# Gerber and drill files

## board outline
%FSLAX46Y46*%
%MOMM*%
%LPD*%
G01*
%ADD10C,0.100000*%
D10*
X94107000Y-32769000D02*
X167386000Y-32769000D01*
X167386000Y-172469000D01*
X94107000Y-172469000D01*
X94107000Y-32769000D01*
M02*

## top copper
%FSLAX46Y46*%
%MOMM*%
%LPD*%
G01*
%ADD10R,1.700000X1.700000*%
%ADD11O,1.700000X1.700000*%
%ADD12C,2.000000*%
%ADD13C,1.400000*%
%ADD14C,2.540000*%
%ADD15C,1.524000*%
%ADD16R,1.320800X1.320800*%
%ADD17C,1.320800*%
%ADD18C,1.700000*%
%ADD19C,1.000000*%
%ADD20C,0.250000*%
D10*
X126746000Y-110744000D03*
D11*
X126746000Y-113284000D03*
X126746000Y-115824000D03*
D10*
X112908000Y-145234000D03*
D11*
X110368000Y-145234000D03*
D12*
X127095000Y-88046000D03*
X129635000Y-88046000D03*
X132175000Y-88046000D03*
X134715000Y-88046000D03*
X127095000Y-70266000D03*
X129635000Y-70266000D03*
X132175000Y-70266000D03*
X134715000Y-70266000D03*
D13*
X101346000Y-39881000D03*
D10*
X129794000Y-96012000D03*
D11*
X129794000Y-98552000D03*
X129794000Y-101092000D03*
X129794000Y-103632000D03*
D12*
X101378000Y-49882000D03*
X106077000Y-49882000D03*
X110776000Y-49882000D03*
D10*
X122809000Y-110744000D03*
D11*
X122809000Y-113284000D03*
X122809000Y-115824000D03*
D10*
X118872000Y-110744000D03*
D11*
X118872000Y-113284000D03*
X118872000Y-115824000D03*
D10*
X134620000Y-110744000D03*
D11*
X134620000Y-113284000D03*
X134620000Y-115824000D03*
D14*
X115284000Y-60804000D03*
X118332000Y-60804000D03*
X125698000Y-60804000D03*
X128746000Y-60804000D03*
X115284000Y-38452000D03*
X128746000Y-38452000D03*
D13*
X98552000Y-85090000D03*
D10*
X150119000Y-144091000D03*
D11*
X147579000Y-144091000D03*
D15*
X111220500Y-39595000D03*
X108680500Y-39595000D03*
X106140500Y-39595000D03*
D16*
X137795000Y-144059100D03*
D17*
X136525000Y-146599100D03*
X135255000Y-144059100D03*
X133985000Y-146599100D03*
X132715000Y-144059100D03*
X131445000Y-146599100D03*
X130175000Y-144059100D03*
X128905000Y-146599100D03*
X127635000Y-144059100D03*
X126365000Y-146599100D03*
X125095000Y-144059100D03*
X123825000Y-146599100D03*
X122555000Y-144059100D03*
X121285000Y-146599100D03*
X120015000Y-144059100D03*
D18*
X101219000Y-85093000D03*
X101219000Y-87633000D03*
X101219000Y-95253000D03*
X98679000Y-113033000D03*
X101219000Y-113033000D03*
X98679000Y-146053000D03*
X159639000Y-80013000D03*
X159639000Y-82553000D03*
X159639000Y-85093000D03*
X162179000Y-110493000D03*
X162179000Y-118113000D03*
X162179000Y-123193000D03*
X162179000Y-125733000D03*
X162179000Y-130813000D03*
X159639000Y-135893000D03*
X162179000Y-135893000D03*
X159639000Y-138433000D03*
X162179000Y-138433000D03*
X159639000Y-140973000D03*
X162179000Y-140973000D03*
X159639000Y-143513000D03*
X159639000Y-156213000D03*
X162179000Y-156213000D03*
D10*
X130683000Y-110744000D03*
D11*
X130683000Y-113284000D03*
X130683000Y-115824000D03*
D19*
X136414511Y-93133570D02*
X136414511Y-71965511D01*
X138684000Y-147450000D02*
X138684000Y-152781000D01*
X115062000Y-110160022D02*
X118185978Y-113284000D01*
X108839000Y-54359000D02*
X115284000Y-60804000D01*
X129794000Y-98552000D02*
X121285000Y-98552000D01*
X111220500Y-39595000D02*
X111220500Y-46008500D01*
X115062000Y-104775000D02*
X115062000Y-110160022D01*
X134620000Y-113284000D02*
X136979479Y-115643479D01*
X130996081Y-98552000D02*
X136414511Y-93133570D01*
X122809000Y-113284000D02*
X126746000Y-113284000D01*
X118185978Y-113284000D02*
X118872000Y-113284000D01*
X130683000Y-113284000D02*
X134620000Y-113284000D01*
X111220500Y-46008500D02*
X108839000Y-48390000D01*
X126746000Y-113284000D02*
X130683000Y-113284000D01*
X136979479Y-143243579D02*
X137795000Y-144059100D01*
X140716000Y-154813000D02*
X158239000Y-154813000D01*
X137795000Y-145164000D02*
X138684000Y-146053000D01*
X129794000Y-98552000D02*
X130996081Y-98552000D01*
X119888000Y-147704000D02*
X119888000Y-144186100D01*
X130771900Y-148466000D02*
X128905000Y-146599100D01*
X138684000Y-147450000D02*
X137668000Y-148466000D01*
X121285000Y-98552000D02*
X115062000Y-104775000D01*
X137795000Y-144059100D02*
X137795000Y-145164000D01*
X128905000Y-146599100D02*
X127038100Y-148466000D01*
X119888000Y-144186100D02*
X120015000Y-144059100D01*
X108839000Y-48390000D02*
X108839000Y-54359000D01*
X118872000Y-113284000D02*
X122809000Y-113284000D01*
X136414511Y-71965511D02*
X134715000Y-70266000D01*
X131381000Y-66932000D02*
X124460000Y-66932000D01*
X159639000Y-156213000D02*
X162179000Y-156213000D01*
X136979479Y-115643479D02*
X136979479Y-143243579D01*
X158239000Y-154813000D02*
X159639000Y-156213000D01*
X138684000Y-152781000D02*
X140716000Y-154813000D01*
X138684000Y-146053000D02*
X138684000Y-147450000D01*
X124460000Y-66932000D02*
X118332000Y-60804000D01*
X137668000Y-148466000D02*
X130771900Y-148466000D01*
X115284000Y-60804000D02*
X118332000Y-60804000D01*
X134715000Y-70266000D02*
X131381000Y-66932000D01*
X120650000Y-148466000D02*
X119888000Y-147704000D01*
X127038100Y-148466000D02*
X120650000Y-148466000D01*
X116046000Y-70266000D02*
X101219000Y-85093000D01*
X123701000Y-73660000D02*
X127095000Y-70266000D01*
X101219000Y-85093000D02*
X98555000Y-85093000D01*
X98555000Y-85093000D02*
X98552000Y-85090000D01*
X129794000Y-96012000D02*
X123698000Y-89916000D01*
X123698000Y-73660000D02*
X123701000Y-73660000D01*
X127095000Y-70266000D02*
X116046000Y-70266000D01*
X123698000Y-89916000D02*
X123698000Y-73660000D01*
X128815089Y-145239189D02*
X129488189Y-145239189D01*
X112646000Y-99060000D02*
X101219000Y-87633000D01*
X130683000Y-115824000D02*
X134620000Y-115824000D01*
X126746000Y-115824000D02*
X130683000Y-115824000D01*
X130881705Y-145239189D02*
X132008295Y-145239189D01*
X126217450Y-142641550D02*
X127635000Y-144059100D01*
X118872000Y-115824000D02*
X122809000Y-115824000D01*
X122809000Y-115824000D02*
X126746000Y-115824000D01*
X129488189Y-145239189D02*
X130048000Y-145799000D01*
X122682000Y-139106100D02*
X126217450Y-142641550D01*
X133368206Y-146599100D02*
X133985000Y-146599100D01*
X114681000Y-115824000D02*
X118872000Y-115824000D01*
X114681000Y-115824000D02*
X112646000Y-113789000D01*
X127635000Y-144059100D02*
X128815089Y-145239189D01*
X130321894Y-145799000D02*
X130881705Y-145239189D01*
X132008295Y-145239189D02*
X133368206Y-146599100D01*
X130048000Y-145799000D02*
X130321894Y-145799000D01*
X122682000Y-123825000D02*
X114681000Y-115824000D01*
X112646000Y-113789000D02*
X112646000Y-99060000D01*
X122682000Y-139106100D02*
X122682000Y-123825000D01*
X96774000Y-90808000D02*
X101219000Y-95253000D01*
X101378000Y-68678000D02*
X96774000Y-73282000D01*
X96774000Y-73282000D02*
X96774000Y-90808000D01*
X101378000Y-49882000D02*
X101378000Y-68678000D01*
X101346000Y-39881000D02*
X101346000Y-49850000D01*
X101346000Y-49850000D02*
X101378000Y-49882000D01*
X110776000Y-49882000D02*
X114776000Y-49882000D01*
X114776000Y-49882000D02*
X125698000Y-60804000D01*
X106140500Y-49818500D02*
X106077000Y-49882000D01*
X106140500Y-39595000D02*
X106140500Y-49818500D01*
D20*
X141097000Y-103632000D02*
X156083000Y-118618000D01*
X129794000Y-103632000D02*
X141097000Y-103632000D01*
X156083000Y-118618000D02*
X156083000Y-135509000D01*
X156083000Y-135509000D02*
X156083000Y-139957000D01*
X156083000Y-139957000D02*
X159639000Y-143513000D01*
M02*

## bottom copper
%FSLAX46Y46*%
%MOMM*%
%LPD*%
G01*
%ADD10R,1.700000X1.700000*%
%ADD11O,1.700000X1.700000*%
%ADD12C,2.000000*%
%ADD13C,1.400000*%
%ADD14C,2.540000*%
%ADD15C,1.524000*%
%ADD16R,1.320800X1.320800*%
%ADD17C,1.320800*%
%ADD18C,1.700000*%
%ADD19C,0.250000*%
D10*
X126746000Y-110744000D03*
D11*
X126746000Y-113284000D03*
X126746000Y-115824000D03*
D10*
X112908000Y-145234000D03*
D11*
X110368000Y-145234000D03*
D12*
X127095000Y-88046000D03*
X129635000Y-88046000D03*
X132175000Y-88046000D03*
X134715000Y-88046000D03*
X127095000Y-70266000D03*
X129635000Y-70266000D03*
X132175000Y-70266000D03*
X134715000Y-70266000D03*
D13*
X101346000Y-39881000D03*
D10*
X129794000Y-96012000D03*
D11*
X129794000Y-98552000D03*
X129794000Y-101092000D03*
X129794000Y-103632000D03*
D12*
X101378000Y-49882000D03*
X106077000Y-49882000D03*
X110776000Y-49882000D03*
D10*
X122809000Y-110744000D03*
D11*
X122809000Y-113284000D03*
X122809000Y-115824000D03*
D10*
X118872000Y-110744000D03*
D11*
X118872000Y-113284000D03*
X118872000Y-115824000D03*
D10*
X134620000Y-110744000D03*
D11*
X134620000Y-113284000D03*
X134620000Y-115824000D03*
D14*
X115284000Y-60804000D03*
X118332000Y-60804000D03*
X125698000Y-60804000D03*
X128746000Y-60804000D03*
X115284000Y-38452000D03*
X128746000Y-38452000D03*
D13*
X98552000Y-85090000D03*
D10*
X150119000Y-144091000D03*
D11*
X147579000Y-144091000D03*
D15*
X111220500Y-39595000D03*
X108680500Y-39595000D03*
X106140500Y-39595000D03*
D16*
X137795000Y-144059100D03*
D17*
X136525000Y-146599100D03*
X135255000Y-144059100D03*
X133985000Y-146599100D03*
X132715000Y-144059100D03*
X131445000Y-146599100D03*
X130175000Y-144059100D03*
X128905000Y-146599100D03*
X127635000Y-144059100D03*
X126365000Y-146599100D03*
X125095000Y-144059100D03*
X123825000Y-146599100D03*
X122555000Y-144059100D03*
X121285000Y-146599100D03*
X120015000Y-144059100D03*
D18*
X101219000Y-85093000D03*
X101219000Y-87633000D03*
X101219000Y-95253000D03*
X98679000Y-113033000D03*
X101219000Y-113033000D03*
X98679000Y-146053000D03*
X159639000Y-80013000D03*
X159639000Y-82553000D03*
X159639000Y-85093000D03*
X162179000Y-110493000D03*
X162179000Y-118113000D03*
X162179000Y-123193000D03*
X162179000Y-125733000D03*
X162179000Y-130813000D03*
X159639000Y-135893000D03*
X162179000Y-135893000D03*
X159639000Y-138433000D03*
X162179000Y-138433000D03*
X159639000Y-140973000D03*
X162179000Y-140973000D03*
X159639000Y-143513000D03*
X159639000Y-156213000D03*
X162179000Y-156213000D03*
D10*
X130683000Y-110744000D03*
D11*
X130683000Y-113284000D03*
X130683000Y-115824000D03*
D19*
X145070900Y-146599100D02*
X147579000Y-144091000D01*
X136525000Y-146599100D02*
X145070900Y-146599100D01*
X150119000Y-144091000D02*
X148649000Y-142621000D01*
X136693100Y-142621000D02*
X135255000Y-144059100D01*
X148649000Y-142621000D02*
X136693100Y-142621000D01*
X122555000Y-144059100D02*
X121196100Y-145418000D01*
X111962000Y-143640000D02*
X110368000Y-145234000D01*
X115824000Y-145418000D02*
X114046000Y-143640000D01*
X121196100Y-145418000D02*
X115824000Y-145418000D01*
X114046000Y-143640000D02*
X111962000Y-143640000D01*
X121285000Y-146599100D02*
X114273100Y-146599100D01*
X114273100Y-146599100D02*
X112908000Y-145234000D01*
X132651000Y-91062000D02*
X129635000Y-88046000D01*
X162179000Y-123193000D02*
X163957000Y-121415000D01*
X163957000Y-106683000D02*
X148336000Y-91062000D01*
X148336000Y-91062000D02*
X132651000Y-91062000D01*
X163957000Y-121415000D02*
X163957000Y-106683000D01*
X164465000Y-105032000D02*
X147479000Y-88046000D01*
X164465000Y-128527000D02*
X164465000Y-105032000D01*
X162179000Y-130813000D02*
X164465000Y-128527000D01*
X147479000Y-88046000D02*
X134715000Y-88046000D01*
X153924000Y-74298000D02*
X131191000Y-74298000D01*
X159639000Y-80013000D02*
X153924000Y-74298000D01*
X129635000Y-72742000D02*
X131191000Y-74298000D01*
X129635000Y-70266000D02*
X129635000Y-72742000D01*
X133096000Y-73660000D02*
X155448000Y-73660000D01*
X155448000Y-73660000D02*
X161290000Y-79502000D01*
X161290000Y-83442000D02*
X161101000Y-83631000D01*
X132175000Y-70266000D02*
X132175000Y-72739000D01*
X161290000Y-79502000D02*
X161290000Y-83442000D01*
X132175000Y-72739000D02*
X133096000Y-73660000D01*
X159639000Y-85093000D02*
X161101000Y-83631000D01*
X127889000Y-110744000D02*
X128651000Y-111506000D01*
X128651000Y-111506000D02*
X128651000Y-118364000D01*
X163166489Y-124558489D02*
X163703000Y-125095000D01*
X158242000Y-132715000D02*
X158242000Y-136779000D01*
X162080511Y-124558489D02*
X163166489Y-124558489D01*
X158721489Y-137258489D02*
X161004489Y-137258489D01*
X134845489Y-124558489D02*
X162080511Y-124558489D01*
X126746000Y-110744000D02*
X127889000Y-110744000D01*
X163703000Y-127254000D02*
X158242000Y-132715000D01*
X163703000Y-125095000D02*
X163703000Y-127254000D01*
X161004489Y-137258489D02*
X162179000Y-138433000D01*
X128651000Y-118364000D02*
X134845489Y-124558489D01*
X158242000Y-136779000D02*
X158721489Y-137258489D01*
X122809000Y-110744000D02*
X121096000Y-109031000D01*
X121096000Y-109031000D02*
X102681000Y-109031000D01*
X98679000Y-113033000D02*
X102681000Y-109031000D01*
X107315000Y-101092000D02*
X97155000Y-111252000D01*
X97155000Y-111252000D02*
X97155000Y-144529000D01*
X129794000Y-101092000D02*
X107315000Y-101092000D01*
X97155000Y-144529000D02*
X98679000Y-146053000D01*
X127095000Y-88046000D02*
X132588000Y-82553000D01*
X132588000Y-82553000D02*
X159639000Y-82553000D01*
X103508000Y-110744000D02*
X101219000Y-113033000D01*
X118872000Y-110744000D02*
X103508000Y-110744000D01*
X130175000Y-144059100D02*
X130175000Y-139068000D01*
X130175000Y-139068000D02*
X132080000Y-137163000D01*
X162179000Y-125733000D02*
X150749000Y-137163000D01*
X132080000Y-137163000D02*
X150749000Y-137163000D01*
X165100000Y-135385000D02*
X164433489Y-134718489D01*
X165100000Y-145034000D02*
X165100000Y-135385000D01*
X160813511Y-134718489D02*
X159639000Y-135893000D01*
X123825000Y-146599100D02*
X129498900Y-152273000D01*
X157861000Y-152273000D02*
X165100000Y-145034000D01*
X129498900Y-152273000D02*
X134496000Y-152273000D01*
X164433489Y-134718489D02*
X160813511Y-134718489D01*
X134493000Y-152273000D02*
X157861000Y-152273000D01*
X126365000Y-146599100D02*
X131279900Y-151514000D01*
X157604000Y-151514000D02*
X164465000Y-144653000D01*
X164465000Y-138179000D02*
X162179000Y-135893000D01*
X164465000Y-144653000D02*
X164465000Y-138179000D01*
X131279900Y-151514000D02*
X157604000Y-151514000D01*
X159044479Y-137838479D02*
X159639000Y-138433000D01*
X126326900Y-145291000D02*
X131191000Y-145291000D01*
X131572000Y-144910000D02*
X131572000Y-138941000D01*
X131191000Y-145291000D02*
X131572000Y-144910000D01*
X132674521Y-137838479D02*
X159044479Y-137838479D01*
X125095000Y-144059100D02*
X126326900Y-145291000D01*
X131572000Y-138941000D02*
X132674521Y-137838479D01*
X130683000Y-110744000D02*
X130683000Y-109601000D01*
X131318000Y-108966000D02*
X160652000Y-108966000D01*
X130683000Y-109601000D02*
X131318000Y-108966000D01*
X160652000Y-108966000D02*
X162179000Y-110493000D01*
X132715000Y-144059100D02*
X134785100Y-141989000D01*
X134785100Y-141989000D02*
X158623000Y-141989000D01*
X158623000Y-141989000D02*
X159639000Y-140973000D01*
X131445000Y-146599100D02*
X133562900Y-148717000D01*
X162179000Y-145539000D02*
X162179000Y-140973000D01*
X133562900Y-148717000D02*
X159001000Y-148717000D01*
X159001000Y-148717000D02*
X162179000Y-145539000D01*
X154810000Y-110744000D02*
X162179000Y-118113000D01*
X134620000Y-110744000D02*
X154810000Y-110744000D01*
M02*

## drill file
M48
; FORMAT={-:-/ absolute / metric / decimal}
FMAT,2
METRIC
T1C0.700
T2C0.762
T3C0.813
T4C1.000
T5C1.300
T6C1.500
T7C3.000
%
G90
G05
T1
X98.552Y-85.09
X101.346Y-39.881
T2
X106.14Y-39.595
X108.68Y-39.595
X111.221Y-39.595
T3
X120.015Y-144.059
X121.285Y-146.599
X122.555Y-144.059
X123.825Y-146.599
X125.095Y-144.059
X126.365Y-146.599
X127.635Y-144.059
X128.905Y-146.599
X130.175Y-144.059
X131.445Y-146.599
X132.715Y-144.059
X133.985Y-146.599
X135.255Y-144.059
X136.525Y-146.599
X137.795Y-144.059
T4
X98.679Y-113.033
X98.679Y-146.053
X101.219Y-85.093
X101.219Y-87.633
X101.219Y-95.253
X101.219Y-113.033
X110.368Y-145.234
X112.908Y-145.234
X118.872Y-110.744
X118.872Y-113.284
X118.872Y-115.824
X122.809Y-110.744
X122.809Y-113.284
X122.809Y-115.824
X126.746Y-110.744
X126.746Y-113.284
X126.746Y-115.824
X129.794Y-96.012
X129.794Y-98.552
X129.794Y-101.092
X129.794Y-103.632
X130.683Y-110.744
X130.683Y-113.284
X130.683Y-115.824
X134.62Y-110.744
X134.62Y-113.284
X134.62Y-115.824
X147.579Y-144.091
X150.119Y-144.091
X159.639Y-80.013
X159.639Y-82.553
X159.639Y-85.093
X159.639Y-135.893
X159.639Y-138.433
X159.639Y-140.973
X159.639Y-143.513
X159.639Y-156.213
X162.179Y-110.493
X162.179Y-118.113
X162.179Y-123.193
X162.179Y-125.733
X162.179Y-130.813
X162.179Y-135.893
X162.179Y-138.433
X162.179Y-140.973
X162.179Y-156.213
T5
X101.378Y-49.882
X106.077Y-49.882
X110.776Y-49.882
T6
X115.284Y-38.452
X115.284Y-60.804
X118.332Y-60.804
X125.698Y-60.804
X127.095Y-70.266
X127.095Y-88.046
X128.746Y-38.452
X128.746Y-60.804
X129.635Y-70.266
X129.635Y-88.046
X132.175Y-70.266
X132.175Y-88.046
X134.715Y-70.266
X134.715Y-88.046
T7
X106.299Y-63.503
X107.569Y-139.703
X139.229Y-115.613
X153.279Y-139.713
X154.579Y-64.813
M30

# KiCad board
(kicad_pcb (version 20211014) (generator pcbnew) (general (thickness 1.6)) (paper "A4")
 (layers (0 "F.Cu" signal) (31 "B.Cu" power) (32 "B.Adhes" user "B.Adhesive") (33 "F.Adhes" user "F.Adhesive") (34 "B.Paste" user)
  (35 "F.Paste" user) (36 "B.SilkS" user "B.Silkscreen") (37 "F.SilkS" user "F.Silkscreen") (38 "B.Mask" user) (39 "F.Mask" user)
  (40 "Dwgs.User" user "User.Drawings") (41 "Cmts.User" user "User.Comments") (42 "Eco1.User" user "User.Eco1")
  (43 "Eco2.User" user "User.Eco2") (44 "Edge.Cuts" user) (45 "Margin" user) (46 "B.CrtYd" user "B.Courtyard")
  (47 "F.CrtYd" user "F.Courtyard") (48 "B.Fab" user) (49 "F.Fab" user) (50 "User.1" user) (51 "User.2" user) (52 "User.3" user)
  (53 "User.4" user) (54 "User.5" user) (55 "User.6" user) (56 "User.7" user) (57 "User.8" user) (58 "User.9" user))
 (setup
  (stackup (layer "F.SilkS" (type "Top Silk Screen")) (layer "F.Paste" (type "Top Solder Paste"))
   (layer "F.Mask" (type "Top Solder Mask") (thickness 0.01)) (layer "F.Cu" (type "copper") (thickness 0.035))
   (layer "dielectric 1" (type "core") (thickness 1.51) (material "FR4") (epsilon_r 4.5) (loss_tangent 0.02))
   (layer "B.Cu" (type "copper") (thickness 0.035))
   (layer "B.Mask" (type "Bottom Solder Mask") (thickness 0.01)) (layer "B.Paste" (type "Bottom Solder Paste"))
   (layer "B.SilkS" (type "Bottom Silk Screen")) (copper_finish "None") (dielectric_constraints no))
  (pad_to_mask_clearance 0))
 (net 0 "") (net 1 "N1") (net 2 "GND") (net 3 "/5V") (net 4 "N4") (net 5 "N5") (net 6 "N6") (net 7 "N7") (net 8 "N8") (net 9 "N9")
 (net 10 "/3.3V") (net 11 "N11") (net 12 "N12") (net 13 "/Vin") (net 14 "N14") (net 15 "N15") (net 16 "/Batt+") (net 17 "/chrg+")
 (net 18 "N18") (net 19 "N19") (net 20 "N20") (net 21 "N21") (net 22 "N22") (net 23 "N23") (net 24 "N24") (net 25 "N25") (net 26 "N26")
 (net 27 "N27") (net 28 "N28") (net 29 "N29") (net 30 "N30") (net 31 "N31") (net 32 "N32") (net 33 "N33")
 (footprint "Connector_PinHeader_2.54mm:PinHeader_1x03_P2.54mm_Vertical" (layer "F.Cu") (at 126.746 110.744)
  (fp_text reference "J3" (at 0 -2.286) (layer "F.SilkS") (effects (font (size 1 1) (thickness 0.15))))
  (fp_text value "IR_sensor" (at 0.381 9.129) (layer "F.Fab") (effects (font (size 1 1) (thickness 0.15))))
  (pad "1" thru_hole rect (at 0 0) (size 1.7 1.7) (drill 1) (layers *.Cu *.Mask) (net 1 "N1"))
  (pad "2" thru_hole oval (at 0 2.54) (size 1.7 1.7) (drill 1) (layers *.Cu *.Mask) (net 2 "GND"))
  (pad "3" thru_hole oval (at 0 5.08) (size 1.7 1.7) (drill 1) (layers *.Cu *.Mask) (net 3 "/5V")))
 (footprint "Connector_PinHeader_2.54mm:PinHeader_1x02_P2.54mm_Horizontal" (layer "F.Cu") (at 112.908 145.234 -90)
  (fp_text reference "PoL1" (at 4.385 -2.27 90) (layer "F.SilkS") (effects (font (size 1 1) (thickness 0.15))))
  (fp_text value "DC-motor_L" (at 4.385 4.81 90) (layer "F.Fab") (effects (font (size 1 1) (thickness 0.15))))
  (pad "1" thru_hole rect (at 0 0 270) (size 1.7 1.7) (drill 1) (layers *.Cu *.Mask) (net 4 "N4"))
  (pad "2" thru_hole oval (at 0 2.54 270) (size 1.7 1.7) (drill 1) (layers *.Cu *.Mask) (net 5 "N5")))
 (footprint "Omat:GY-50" (layer "F.Cu") (at 119.348 90.713)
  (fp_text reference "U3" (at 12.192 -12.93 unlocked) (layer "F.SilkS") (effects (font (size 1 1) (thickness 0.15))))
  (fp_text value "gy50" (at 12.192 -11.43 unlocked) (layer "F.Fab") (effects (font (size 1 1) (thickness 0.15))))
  (pad "1" thru_hole circle (at 7.747 -2.667) (size 2 2) (drill 1.5) (layers *.Cu *.Mask) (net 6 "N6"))
  (pad "2" thru_hole circle (at 10.287 -2.667) (size 2 2) (drill 1.5) (layers *.Cu *.Mask) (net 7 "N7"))
  (pad "3" thru_hole circle (at 12.827 -2.667) (size 2 2) (drill 1.5) (layers *.Cu *.Mask) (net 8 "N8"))
  (pad "4" thru_hole circle (at 15.367 -2.667) (size 2 2) (drill 1.5) (layers *.Cu *.Mask) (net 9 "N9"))
  (pad "5" thru_hole circle (at 7.747 -20.447) (size 2 2) (drill 1.5) (layers *.Cu *.Mask) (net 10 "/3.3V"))
  (pad "6" thru_hole circle (at 10.287 -20.447) (size 2 2) (drill 1.5) (layers *.Cu *.Mask) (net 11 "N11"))
  (pad "7" thru_hole circle (at 12.827 -20.447) (size 2 2) (drill 1.5) (layers *.Cu *.Mask) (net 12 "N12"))
  (pad "8" thru_hole circle (at 15.367 -20.447) (size 2 2) (drill 1.5) (layers *.Cu *.Mask) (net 2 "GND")))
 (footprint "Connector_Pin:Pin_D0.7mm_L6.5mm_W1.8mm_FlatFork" (layer "F.Cu") (at 101.346 39.881)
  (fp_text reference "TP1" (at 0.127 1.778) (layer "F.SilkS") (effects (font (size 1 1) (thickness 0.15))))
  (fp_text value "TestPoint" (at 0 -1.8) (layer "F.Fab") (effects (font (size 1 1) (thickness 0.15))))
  (pad "1" thru_hole circle (at 0 0) (size 1.4 1.4) (drill 0.7) (layers *.Cu *.Mask) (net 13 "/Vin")))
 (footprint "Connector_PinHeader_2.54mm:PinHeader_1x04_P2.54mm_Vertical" (layer "F.Cu") (at 129.794 96.012)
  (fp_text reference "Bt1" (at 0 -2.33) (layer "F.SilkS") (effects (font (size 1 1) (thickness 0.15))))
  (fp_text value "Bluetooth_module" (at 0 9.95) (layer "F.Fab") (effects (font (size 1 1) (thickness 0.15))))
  (pad "1" thru_hole rect (at 0 0) (size 1.7 1.7) (drill 1) (layers *.Cu *.Mask) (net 10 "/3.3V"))
  (pad "2" thru_hole oval (at 0 2.54) (size 1.7 1.7) (drill 1) (layers *.Cu *.Mask) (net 2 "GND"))
  (pad "3" thru_hole oval (at 0 5.08) (size 1.7 1.7) (drill 1) (layers *.Cu *.Mask) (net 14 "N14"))
  (pad "4" thru_hole oval (at 0 7.62) (size 1.7 1.7) (drill 1) (layers *.Cu *.Mask) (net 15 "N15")))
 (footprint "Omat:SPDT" (layer "F.Cu") (at 112.681 45.818 180)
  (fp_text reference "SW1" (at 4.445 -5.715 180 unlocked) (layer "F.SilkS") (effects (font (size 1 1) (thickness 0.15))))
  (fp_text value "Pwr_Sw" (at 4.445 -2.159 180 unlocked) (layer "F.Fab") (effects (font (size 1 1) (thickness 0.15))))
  (pad "1" thru_hole circle (at 11.303 -4.064 180) (size 2 2) (drill 1.3) (layers *.Cu *.Mask) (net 13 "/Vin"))
  (pad "2" thru_hole circle (at 6.604 -4.064 180) (size 2 2) (drill 1.3) (layers *.Cu *.Mask) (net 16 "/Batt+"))
  (pad "3" thru_hole circle (at 1.905 -4.064 180) (size 2 2) (drill 1.3) (layers *.Cu *.Mask) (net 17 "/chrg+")))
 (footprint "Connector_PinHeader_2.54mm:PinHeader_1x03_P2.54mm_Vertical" (layer "F.Cu") (at 122.809 110.744)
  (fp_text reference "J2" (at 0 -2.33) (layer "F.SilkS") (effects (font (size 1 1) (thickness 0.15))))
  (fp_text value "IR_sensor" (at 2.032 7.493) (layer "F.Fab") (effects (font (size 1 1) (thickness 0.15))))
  (pad "1" thru_hole rect (at 0 0) (size 1.7 1.7) (drill 1) (layers *.Cu *.Mask) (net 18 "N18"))
  (pad "2" thru_hole oval (at 0 2.54) (size 1.7 1.7) (drill 1) (layers *.Cu *.Mask) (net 2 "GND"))
  (pad "3" thru_hole oval (at 0 5.08) (size 1.7 1.7) (drill 1) (layers *.Cu *.Mask) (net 3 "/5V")))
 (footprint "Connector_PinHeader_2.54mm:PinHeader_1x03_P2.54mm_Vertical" (layer "F.Cu") (at 118.872 110.744)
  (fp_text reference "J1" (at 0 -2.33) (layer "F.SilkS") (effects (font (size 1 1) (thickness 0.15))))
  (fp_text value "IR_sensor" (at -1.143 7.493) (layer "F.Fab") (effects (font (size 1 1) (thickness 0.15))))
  (pad "1" thru_hole rect (at 0 0) (size 1.7 1.7) (drill 1) (layers *.Cu *.Mask) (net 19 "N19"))
  (pad "2" thru_hole oval (at 0 2.54) (size 1.7 1.7) (drill 1) (layers *.Cu *.Mask) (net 2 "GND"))
  (pad "3" thru_hole oval (at 0 5.08) (size 1.7 1.7) (drill 1) (layers *.Cu *.Mask) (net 3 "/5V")))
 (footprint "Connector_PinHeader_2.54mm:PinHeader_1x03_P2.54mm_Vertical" (layer "F.Cu") (at 134.62 110.744)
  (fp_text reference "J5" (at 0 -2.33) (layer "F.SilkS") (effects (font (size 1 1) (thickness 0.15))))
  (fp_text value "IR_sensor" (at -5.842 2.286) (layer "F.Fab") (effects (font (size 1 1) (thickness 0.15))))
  (pad "1" thru_hole rect (at 0 0) (size 1.7 1.7) (drill 1) (layers *.Cu *.Mask) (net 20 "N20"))
  (pad "2" thru_hole oval (at 0 2.54) (size 1.7 1.7) (drill 1) (layers *.Cu *.Mask) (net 2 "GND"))
  (pad "3" thru_hole oval (at 0 5.08) (size 1.7 1.7) (drill 1) (layers *.Cu *.Mask) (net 3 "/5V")))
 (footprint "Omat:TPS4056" (layer "F.Cu") (at 113.506 35.912 -90)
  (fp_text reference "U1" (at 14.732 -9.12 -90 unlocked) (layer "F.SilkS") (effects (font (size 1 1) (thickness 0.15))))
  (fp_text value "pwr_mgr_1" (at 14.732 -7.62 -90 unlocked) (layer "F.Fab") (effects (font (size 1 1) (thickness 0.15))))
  (pad "1" thru_hole circle (at 24.892 -1.778 270) (size 2.54 2.54) (drill 1.5) (layers *.Cu *.Mask) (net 2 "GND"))
  (pad "2" thru_hole circle (at 24.892 -4.826 270) (size 2.54 2.54) (drill 1.5) (layers *.Cu *.Mask) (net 2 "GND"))
  (pad "3" thru_hole circle (at 24.892 -12.192 270) (size 2.54 2.54) (drill 1.5) (layers *.Cu *.Mask) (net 17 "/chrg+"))
  (pad "4" thru_hole circle (at 24.892 -15.24 270) (size 2.54 2.54) (drill 1.5) (layers *.Cu *.Mask) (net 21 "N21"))
  (pad "5" thru_hole circle (at 2.54 -1.778 270) (size 2.54 2.54) (drill 1.5) (layers *.Cu *.Mask) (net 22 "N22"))
  (pad "6" thru_hole circle (at 2.54 -15.24 270) (size 2.54 2.54) (drill 1.5) (layers *.Cu *.Mask) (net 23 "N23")))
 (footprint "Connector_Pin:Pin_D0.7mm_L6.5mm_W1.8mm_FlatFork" (layer "F.Cu") (at 98.552 85.09)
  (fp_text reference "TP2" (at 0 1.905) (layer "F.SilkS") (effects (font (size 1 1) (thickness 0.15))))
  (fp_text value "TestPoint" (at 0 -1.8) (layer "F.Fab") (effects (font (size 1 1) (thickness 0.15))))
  (pad "1" thru_hole circle (at 0 0) (size 1.4 1.4) (drill 0.7) (layers *.Cu *.Mask) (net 10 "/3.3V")))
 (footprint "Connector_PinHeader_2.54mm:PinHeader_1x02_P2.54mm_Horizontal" (layer "F.Cu") (at 150.119 144.091 -90)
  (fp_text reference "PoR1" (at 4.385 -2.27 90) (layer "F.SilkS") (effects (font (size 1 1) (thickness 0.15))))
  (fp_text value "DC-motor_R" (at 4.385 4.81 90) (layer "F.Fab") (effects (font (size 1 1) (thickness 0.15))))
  (pad "1" thru_hole rect (at 0 0 270) (size 1.7 1.7) (drill 1) (layers *.Cu *.Mask) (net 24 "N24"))
  (pad "2" thru_hole oval (at 0 2.54 270) (size 1.7 1.7) (drill 1) (layers *.Cu *.Mask) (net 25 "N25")))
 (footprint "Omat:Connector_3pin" (layer "F.Cu") (at 112.3635 38.325 180)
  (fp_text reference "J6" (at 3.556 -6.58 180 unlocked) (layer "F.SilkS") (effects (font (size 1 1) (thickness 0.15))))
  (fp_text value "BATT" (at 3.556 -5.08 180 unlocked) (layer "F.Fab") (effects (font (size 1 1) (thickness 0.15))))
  (pad "1" thru_hole circle (at 1.143 -1.27 180) (size 1.524 1.524) (drill 0.762) (layers *.Cu *.Mask) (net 2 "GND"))
  (pad "2" thru_hole circle (at 3.683 -1.27 180) (size 1.524 1.524) (drill 0.762) (layers *.Cu *.Mask) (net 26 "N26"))
  (pad "3" thru_hole circle (at 6.223 -1.27 180) (size 1.524 1.524) (drill 0.762) (layers *.Cu *.Mask) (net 16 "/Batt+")))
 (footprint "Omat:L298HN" (layer "F.Cu") (at 137.795 144.0591 180)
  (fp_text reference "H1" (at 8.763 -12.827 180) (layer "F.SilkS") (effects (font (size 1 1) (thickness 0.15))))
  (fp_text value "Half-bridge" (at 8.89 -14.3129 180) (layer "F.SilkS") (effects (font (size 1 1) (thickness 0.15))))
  (pad "1" thru_hole rect (at 0 0 180) (size 1.3208 1.3208) (drill 0.8128) (layers *.Cu *.Mask) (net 2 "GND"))
  (pad "2" thru_hole circle (at 1.27 -2.54 180) (size 1.3208 1.3208) (drill 0.8128) (layers *.Cu *.Mask) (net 25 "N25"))
  (pad "3" thru_hole circle (at 2.54 0 180) (size 1.3208 1.3208) (drill 0.8128) (layers *.Cu *.Mask) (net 24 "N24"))
  (pad "4" thru_hole circle (at 3.81 -2.54 180) (size 1.3208 1.3208) (drill 0.8128) (layers *.Cu *.Mask) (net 3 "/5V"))
  (pad "5" thru_hole circle (at 5.08 0 180) (size 1.3208 1.3208) (drill 0.8128) (layers *.Cu *.Mask) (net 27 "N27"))
  (pad "6" thru_hole circle (at 6.35 -2.54 180) (size 1.3208 1.3208) (drill 0.8128) (layers *.Cu *.Mask) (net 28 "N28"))
  (pad "7" thru_hole circle (at 7.62 0 180) (size 1.3208 1.3208) (drill 0.8128) (layers *.Cu *.Mask) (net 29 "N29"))
  (pad "8" thru_hole circle (at 8.89 -2.54 180) (size 1.3208 1.3208) (drill 0.8128) (layers *.Cu *.Mask) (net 2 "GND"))
  (pad "9" thru_hole circle (at 10.16 0 180) (size 1.3208 1.3208) (drill 0.8128) (layers *.Cu *.Mask) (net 3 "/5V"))
  (pad "10" thru_hole circle (at 11.43 -2.54 180) (size 1.3208 1.3208) (drill 0.8128) (layers *.Cu *.Mask) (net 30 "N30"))
  (pad "11" thru_hole circle (at 12.7 0 180) (size 1.3208 1.3208) (drill 0.8128) (layers *.Cu *.Mask) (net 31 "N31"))
  (pad "12" thru_hole circle (at 13.97 -2.54 180) (size 1.3208 1.3208) (drill 0.8128) (layers *.Cu *.Mask) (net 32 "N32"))
  (pad "13" thru_hole circle (at 15.24 0 180) (size 1.3208 1.3208) (drill 0.8128) (layers *.Cu *.Mask) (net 5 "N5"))
  (pad "14" thru_hole circle (at 16.51 -2.54 180) (size 1.3208 1.3208) (drill 0.8128) (layers *.Cu *.Mask) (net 4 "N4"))
  (pad "15" thru_hole circle (at 17.78 0 180) (size 1.3208 1.3208) (drill 0.8128) (layers *.Cu *.Mask) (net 2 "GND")))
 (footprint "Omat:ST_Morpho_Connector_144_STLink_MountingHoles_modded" (layer "F.Cu") (at 98.679 67.313)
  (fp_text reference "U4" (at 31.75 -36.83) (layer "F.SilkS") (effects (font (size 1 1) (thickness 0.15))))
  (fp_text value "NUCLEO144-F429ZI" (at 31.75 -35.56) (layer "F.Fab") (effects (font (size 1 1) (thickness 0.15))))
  (pad "" np_thru_hole circle (at 40.55 48.3) (size 3 3) (drill 3) (layers *.Cu *.Mask))
  (pad "" np_thru_hole circle (at 55.9 -2.5) (size 3 3) (drill 3) (layers *.Cu *.Mask))
  (pad "" np_thru_hole circle (at 8.89 72.39) (size 3 3) (drill 3) (layers *.Cu *.Mask))
  (pad "" np_thru_hole circle (at 7.62 -3.81) (size 3 3) (drill 3) (layers *.Cu *.Mask))
  (pad "" np_thru_hole circle (at 54.6 72.4) (size 3 3) (drill 3) (layers *.Cu *.Mask))
  (pad "16" thru_hole circle (at 2.54 17.78) (size 1.7 1.7) (drill 1) (layers *.Cu *.Mask) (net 10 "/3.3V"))
  (pad "18" thru_hole circle (at 2.54 20.32) (size 1.7 1.7) (drill 1) (layers *.Cu *.Mask) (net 3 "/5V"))
  (pad "24" thru_hole circle (at 2.54 27.94) (size 1.7 1.7) (drill 1) (layers *.Cu *.Mask) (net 13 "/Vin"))
  (pad "37" thru_hole circle (at 0 45.72) (size 1.7 1.7) (drill 1) (layers *.Cu *.Mask) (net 18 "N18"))
  (pad "38" thru_hole circle (at 2.54 45.72) (size 1.7 1.7) (drill 1) (layers *.Cu *.Mask) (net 19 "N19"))
  (pad "63" thru_hole circle (at 0 78.74) (size 1.7 1.7) (drill 1) (layers *.Cu *.Mask) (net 14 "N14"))
  (pad "83" thru_hole circle (at 60.96 12.7) (size 1.7 1.7) (drill 1) (layers *.Cu *.Mask) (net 11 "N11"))
  (pad "85" thru_hole circle (at 60.96 15.24) (size 1.7 1.7) (drill 1) (layers *.Cu *.Mask) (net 6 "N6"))
  (pad "87" thru_hole circle (at 60.96 17.78) (size 1.7 1.7) (drill 1) (layers *.Cu *.Mask) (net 12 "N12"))
  (pad "108" thru_hole circle (at 63.5 43.18) (size 1.7 1.7) (drill 1) (layers *.Cu *.Mask) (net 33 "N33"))
  (pad "114" thru_hole circle (at 63.5 50.8) (size 1.7 1.7) (drill 1) (layers *.Cu *.Mask) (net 20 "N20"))
  (pad "118" thru_hole circle (at 63.5 55.88) (size 1.7 1.7) (drill 1) (layers *.Cu *.Mask) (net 7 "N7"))
  (pad "120" thru_hole circle (at 63.5 58.42) (size 1.7 1.7) (drill 1) (layers *.Cu *.Mask) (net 29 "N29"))
  (pad "124" thru_hole circle (at 63.5 63.5) (size 1.7 1.7) (drill 1) (layers *.Cu *.Mask) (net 9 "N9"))
  (pad "127" thru_hole circle (at 60.96 68.58) (size 1.7 1.7) (drill 1) (layers *.Cu *.Mask) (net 32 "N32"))
  (pad "128" thru_hole circle (at 63.5 68.58) (size 1.7 1.7) (drill 1) (layers *.Cu *.Mask) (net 30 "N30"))
  (pad "129" thru_hole circle (at 60.96 71.12) (size 1.7 1.7) (drill 1) (layers *.Cu *.Mask) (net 31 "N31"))
  (pad "130" thru_hole circle (at 63.5 71.12) (size 1.7 1.7) (drill 1) (layers *.Cu *.Mask) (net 1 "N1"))
  (pad "131" thru_hole circle (at 60.96 73.66) (size 1.7 1.7) (drill 1) (layers *.Cu *.Mask) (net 27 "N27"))
  (pad "132" thru_hole circle (at 63.5 73.66) (size 1.7 1.7) (drill 1) (layers *.Cu *.Mask) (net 28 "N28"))
  (pad "133" thru_hole circle (at 60.96 76.2) (size 1.7 1.7) (drill 1) (layers *.Cu *.Mask) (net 15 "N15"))
  (pad "143" thru_hole circle (at 60.96 88.9) (size 1.7 1.7) (drill 1) (layers *.Cu *.Mask) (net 2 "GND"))
  (pad "144" thru_hole circle (at 63.5 88.9) (size 1.7 1.7) (drill 1) (layers *.Cu *.Mask) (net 2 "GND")))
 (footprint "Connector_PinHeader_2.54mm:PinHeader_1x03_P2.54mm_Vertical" (layer "F.Cu") (at 130.683 110.744)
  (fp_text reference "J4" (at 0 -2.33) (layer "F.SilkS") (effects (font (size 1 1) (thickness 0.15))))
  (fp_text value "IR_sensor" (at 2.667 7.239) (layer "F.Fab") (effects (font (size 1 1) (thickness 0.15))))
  (pad "1" thru_hole rect (at 0 0) (size 1.7 1.7) (drill 1) (layers *.Cu *.Mask) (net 33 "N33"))
  (pad "2" thru_hole oval (at 0 2.54) (size 1.7 1.7) (drill 1) (layers *.Cu *.Mask) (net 2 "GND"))
  (pad "3" thru_hole oval (at 0 5.08) (size 1.7 1.7) (drill 1) (layers *.Cu *.Mask) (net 3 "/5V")))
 (gr_rect (start 94.107 32.769) (end 167.386 172.469) (layer "Edge.Cuts") (width 0.1) (fill none))
 (segment (start 136.414511 93.13357) (end 136.414511 71.965511) (width 1) (layer "F.Cu") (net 2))
 (segment (start 138.684 147.45) (end 138.684 152.781) (width 1) (layer "F.Cu") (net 2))
 (segment (start 115.062 110.160022) (end 118.185978 113.284) (width 1) (layer "F.Cu") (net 2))
 (segment (start 108.839 54.359) (end 115.284 60.804) (width 1) (layer "F.Cu") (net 2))
 (segment (start 129.794 98.552) (end 121.285 98.552) (width 1) (layer "F.Cu") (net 2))
 (segment (start 111.2205 39.595) (end 111.2205 46.0085) (width 1) (layer "F.Cu") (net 2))
 (segment (start 115.062 104.775) (end 115.062 110.160022) (width 1) (layer "F.Cu") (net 2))
 (segment (start 134.62 113.284) (end 136.979479 115.643479) (width 1) (layer "F.Cu") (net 2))
 (segment (start 130.996081 98.552) (end 136.414511 93.13357) (width 1) (layer "F.Cu") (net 2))
 (segment (start 122.809 113.284) (end 126.746 113.284) (width 1) (layer "F.Cu") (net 2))
 (segment (start 118.185978 113.284) (end 118.872 113.284) (width 1) (layer "F.Cu") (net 2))
 (segment (start 130.683 113.284) (end 134.62 113.284) (width 1) (layer "F.Cu") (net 2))
 (segment (start 111.2205 46.0085) (end 108.839 48.39) (width 1) (layer "F.Cu") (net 2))
 (segment (start 126.746 113.284) (end 130.683 113.284) (width 1) (layer "F.Cu") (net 2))
 (segment (start 136.979479 143.243579) (end 137.795 144.0591) (width 1) (layer "F.Cu") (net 2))
 (segment (start 140.716 154.813) (end 158.239 154.813) (width 1) (layer "F.Cu") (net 2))
 (segment (start 137.795 145.164) (end 138.684 146.053) (width 1) (layer "F.Cu") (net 2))
 (segment (start 129.794 98.552) (end 130.996081 98.552) (width 1) (layer "F.Cu") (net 2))
 (segment (start 119.888 147.704) (end 119.888 144.1861) (width 1) (layer "F.Cu") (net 2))
 (segment (start 130.7719 148.466) (end 128.905 146.5991) (width 1) (layer "F.Cu") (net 2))
 (segment (start 138.684 147.45) (end 137.668 148.466) (width 1) (layer "F.Cu") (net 2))
 (segment (start 121.285 98.552) (end 115.062 104.775) (width 1) (layer "F.Cu") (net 2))
 (segment (start 137.795 144.0591) (end 137.795 145.164) (width 1) (layer "F.Cu") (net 2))
 (segment (start 128.905 146.5991) (end 127.0381 148.466) (width 1) (layer "F.Cu") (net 2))
 (segment (start 119.888 144.1861) (end 120.015 144.0591) (width 1) (layer "F.Cu") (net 2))
 (segment (start 108.839 48.39) (end 108.839 54.359) (width 1) (layer "F.Cu") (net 2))
 (segment (start 118.872 113.284) (end 122.809 113.284) (width 1) (layer "F.Cu") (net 2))
 (segment (start 136.414511 71.965511) (end 134.715 70.266) (width 1) (layer "F.Cu") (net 2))
 (segment (start 131.381 66.932) (end 124.46 66.932) (width 1) (layer "F.Cu") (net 2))
 (segment (start 159.639 156.213) (end 162.179 156.213) (width 1) (layer "F.Cu") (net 2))
 (segment (start 136.979479 115.643479) (end 136.979479 143.243579) (width 1) (layer "F.Cu") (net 2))
 (segment (start 158.239 154.813) (end 159.639 156.213) (width 1) (layer "F.Cu") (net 2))
 (segment (start 138.684 152.781) (end 140.716 154.813) (width 1) (layer "F.Cu") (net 2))
 (segment (start 138.684 146.053) (end 138.684 147.45) (width 1) (layer "F.Cu") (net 2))
 (segment (start 124.46 66.932) (end 118.332 60.804) (width 1) (layer "F.Cu") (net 2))
 (segment (start 137.668 148.466) (end 130.7719 148.466) (width 1) (layer "F.Cu") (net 2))
 (segment (start 115.284 60.804) (end 118.332 60.804) (width 1) (layer "F.Cu") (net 2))
 (segment (start 134.715 70.266) (end 131.381 66.932) (width 1) (layer "F.Cu") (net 2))
 (segment (start 120.65 148.466) (end 119.888 147.704) (width 1) (layer "F.Cu") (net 2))
 (segment (start 127.0381 148.466) (end 120.65 148.466) (width 1) (layer "F.Cu") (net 2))
 (segment (start 145.0709 146.5991) (end 147.579 144.091) (width 0.25) (layer "B.Cu") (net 25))
 (segment (start 136.525 146.5991) (end 145.0709 146.5991) (width 0.25) (layer "B.Cu") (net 25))
 (segment (start 150.119 144.091) (end 148.649 142.621) (width 0.25) (layer "B.Cu") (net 24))
 (segment (start 136.6931 142.621) (end 135.255 144.0591) (width 0.25) (layer "B.Cu") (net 24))
 (segment (start 148.649 142.621) (end 136.6931 142.621) (width 0.25) (layer "B.Cu") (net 24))
 (segment (start 116.046 70.266) (end 101.219 85.093) (width 1) (layer "F.Cu") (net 10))
 (segment (start 123.701 73.66) (end 127.095 70.266) (width 1) (layer "F.Cu") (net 10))
 (segment (start 101.219 85.093) (end 98.555 85.093) (width 1) (layer "F.Cu") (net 10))
 (segment (start 98.555 85.093) (end 98.552 85.09) (width 1) (layer "F.Cu") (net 10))
 (segment (start 129.794 96.012) (end 123.698 89.916) (width 1) (layer "F.Cu") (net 10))
 (segment (start 123.698 73.66) (end 123.701 73.66) (width 1) (layer "F.Cu") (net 10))
 (segment (start 127.095 70.266) (end 116.046 70.266) (width 1) (layer "F.Cu") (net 10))
 (segment (start 123.698 89.916) (end 123.698 73.66) (width 1) (layer "F.Cu") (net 10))
 (segment (start 122.555 144.0591) (end 121.1961 145.418) (width 0.25) (layer "B.Cu") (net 5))
 (segment (start 111.962 143.64) (end 110.368 145.234) (width 0.25) (layer "B.Cu") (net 5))
 (segment (start 115.824 145.418) (end 114.046 143.64) (width 0.25) (layer "B.Cu") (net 5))
 (segment (start 121.1961 145.418) (end 115.824 145.418) (width 0.25) (layer "B.Cu") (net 5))
 (segment (start 114.046 143.64) (end 111.962 143.64) (width 0.25) (layer "B.Cu") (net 5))
 (segment (start 121.285 146.5991) (end 114.2731 146.5991) (width 0.25) (layer "B.Cu") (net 4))
 (segment (start 114.2731 146.5991) (end 112.908 145.234) (width 0.25) (layer "B.Cu") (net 4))
 (segment (start 132.651 91.062) (end 129.635 88.046) (width 0.25) (layer "B.Cu") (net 7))
 (segment (start 162.179 123.193) (end 163.957 121.415) (width 0.25) (layer "B.Cu") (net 7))
 (segment (start 163.957 106.683) (end 148.336 91.062) (width 0.25) (layer "B.Cu") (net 7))
 (segment (start 148.336 91.062) (end 132.651 91.062) (width 0.25) (layer "B.Cu") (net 7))
 (segment (start 163.957 121.415) (end 163.957 106.683) (width 0.25) (layer "B.Cu") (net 7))
 (segment (start 164.465 105.032) (end 147.479 88.046) (width 0.25) (layer "B.Cu") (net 9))
 (segment (start 164.465 128.527) (end 164.465 105.032) (width 0.25) (layer "B.Cu") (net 9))
 (segment (start 162.179 130.813) (end 164.465 128.527) (width 0.25) (layer "B.Cu") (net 9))
 (segment (start 147.479 88.046) (end 134.715 88.046) (width 0.25) (layer "B.Cu") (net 9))
 (segment (start 153.924 74.298) (end 131.191 74.298) (width 0.25) (layer "B.Cu") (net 11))
 (segment (start 159.639 80.013) (end 153.924 74.298) (width 0.25) (layer "B.Cu") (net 11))
 (segment (start 129.635 72.742) (end 131.191 74.298) (width 0.25) (layer "B.Cu") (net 11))
 (segment (start 129.635 70.266) (end 129.635 72.742) (width 0.25) (layer "B.Cu") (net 11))
 (segment (start 133.096 73.66) (end 155.448 73.66) (width 0.25) (layer "B.Cu") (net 12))
 (segment (start 155.448 73.66) (end 161.29 79.502) (width 0.25) (layer "B.Cu") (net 12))
 (segment (start 161.29 83.442) (end 161.101 83.631) (width 0.25) (layer "B.Cu") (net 12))
 (segment (start 132.175 70.266) (end 132.175 72.739) (width 0.25) (layer "B.Cu") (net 12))
 (segment (start 161.29 79.502) (end 161.29 83.442) (width 0.25) (layer "B.Cu") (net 12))
 (segment (start 132.175 72.739) (end 133.096 73.66) (width 0.25) (layer "B.Cu") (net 12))
 (segment (start 159.639 85.093) (end 161.101 83.631) (width 0.25) (layer "B.Cu") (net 12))
 (segment (start 127.889 110.744) (end 128.651 111.506) (width 0.25) (layer "B.Cu") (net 1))
 (segment (start 128.651 111.506) (end 128.651 118.364) (width 0.25) (layer "B.Cu") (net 1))
 (segment (start 163.166489 124.558489) (end 163.703 125.095) (width 0.25) (layer "B.Cu") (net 1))
 (segment (start 158.242 132.715) (end 158.242 136.779) (width 0.25) (layer "B.Cu") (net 1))
 (segment (start 162.080511 124.558489) (end 163.166489 124.558489) (width 0.25) (layer "B.Cu") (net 1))
 (segment (start 158.721489 137.258489) (end 161.004489 137.258489) (width 0.25) (layer "B.Cu") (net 1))
 (segment (start 134.845489 124.558489) (end 162.080511 124.558489) (width 0.25) (layer "B.Cu") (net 1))
 (segment (start 126.746 110.744) (end 127.889 110.744) (width 0.25) (layer "B.Cu") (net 1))
 (segment (start 163.703 127.254) (end 158.242 132.715) (width 0.25) (layer "B.Cu") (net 1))
 (segment (start 163.703 125.095) (end 163.703 127.254) (width 0.25) (layer "B.Cu") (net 1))
 (segment (start 161.004489 137.258489) (end 162.179 138.433) (width 0.25) (layer "B.Cu") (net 1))
 (segment (start 128.651 118.364) (end 134.845489 124.558489) (width 0.25) (layer "B.Cu") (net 1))
 (segment (start 158.242 136.779) (end 158.721489 137.258489) (width 0.25) (layer "B.Cu") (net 1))
 (segment (start 128.815089 145.239189) (end 129.488189 145.239189) (width 1) (layer "F.Cu") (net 3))
 (segment (start 112.646 99.06) (end 101.219 87.633) (width 1) (layer "F.Cu") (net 3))
 (segment (start 130.683 115.824) (end 134.62 115.824) (width 1) (layer "F.Cu") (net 3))
 (segment (start 126.746 115.824) (end 130.683 115.824) (width 1) (layer "F.Cu") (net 3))
 (segment (start 130.881705 145.239189) (end 132.008295 145.239189) (width 1) (layer "F.Cu") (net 3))
 (segment (start 126.21745 142.64155) (end 127.635 144.0591) (width 1) (layer "F.Cu") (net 3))
 (segment (start 118.872 115.824) (end 122.809 115.824) (width 1) (layer "F.Cu") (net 3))
 (segment (start 122.809 115.824) (end 126.746 115.824) (width 1) (layer "F.Cu") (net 3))
 (segment (start 129.488189 145.239189) (end 130.048 145.799) (width 1) (layer "F.Cu") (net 3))
 (segment (start 122.682 139.1061) (end 126.21745 142.64155) (width 1) (layer "F.Cu") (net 3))
 (segment (start 133.368206 146.5991) (end 133.985 146.5991) (width 1) (layer "F.Cu") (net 3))
 (segment (start 114.681 115.824) (end 118.872 115.824) (width 1) (layer "F.Cu") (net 3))
 (segment (start 114.681 115.824) (end 112.646 113.789) (width 1) (layer "F.Cu") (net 3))
 (segment (start 127.635 144.0591) (end 128.815089 145.239189) (width 1) (layer "F.Cu") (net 3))
 (segment (start 130.321894 145.799) (end 130.881705 145.239189) (width 1) (layer "F.Cu") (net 3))
 (segment (start 132.008295 145.239189) (end 133.368206 146.5991) (width 1) (layer "F.Cu") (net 3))
 (segment (start 130.048 145.799) (end 130.321894 145.799) (width 1) (layer "F.Cu") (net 3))
 (segment (start 122.682 123.825) (end 114.681 115.824) (width 1) (layer "F.Cu") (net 3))
 (segment (start 112.646 113.789) (end 112.646 99.06) (width 1) (layer "F.Cu") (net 3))
 (segment (start 122.682 139.1061) (end 122.682 123.825) (width 1) (layer "F.Cu") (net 3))
 (segment (start 96.774 90.808) (end 101.219 95.253) (width 1) (layer "F.Cu") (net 13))
 (segment (start 101.378 68.678) (end 96.774 73.282) (width 1) (layer "F.Cu") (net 13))
 (segment (start 96.774 73.282) (end 96.774 90.808) (width 1) (layer "F.Cu") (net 13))
 (segment (start 101.378 49.882) (end 101.378 68.678) (width 1) (layer "F.Cu") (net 13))
 (segment (start 101.346 39.881) (end 101.346 49.85) (width 1) (layer "F.Cu") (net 13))
 (segment (start 101.346 49.85) (end 101.378 49.882) (width 1) (layer "F.Cu") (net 13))
 (segment (start 110.776 49.882) (end 114.776 49.882) (width 1) (layer "F.Cu") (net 17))
 (segment (start 114.776 49.882) (end 125.698 60.804) (width 1) (layer "F.Cu") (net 17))
 (segment (start 106.1405 49.8185) (end 106.077 49.882) (width 1) (layer "F.Cu") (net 16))
 (segment (start 106.1405 39.595) (end 106.1405 49.8185) (width 1) (layer "F.Cu") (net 16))
 (segment (start 122.809 110.744) (end 121.096 109.031) (width 0.25) (layer "B.Cu") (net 18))
 (segment (start 121.096 109.031) (end 102.681 109.031) (width 0.25) (layer "B.Cu") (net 18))
 (segment (start 98.679 113.033) (end 102.681 109.031) (width 0.25) (layer "B.Cu") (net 18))
 (segment (start 107.315 101.092) (end 97.155 111.252) (width 0.25) (layer "B.Cu") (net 14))
 (segment (start 97.155 111.252) (end 97.155 144.529) (width 0.25) (layer "B.Cu") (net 14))
 (segment (start 129.794 101.092) (end 107.315 101.092) (width 0.25) (layer "B.Cu") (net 14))
 (segment (start 97.155 144.529) (end 98.679 146.053) (width 0.25) (layer "B.Cu") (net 14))
 (segment (start 127.095 88.046) (end 132.588 82.553) (width 0.25) (layer "B.Cu") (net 6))
 (segment (start 132.588 82.553) (end 159.639 82.553) (width 0.25) (layer "B.Cu") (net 6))
 (segment (start 103.508 110.744) (end 101.219 113.033) (width 0.25) (layer "B.Cu") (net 19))
 (segment (start 118.872 110.744) (end 103.508 110.744) (width 0.25) (layer "B.Cu") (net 19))
 (segment (start 130.175 144.0591) (end 130.175 139.068) (width 0.25) (layer "B.Cu") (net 29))
 (segment (start 130.175 139.068) (end 132.08 137.163) (width 0.25) (layer "B.Cu") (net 29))
 (segment (start 162.179 125.733) (end 150.749 137.163) (width 0.25) (layer "B.Cu") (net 29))
 (segment (start 132.08 137.163) (end 150.749 137.163) (width 0.25) (layer "B.Cu") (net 29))
 (segment (start 165.1 135.385) (end 164.433489 134.718489) (width 0.25) (layer "B.Cu") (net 32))
 (segment (start 165.1 145.034) (end 165.1 135.385) (width 0.25) (layer "B.Cu") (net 32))
 (segment (start 160.813511 134.718489) (end 159.639 135.893) (width 0.25) (layer "B.Cu") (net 32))
 (segment (start 123.825 146.5991) (end 129.4989 152.273) (width 0.25) (layer "B.Cu") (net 32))
 (segment (start 157.861 152.273) (end 165.1 145.034) (width 0.25) (layer "B.Cu") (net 32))
 (segment (start 129.4989 152.273) (end 134.496 152.273) (width 0.25) (layer "B.Cu") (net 32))
 (segment (start 164.433489 134.718489) (end 160.813511 134.718489) (width 0.25) (layer "B.Cu") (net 32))
 (segment (start 134.493 152.273) (end 157.861 152.273) (width 0.25) (layer "B.Cu") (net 32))
 (segment (start 126.365 146.5991) (end 131.2799 151.514) (width 0.25) (layer "B.Cu") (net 30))
 (segment (start 157.604 151.514) (end 164.465 144.653) (width 0.25) (layer "B.Cu") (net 30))
 (segment (start 164.465 138.179) (end 162.179 135.893) (width 0.25) (layer "B.Cu") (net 30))
 (segment (start 164.465 144.653) (end 164.465 138.179) (width 0.25) (layer "B.Cu") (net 30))
 (segment (start 131.2799 151.514) (end 157.604 151.514) (width 0.25) (layer "B.Cu") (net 30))
 (segment (start 159.044479 137.838479) (end 159.639 138.433) (width 0.25) (layer "B.Cu") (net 31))
 (segment (start 126.3269 145.291) (end 131.191 145.291) (width 0.25) (layer "B.Cu") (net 31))
 (segment (start 131.572 144.91) (end 131.572 138.941) (width 0.25) (layer "B.Cu") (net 31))
 (segment (start 131.191 145.291) (end 131.572 144.91) (width 0.25) (layer "B.Cu") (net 31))
 (segment (start 132.674521 137.838479) (end 159.044479 137.838479) (width 0.25) (layer "B.Cu") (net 31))
 (segment (start 125.095 144.0591) (end 126.3269 145.291) (width 0.25) (layer "B.Cu") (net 31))
 (segment (start 131.572 138.941) (end 132.674521 137.838479) (width 0.25) (layer "B.Cu") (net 31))
 (segment (start 130.683 110.744) (end 130.683 109.601) (width 0.25) (layer "B.Cu") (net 33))
 (segment (start 131.318 108.966) (end 160.652 108.966) (width 0.25) (layer "B.Cu") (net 33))
 (segment (start 130.683 109.601) (end 131.318 108.966) (width 0.25) (layer "B.Cu") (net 33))
 (segment (start 160.652 108.966) (end 162.179 110.493) (width 0.25) (layer "B.Cu") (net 33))
 (segment (start 132.715 144.0591) (end 134.7851 141.989) (width 0.25) (layer "B.Cu") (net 27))
 (segment (start 134.7851 141.989) (end 158.623 141.989) (width 0.25) (layer "B.Cu") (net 27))
 (segment (start 158.623 141.989) (end 159.639 140.973) (width 0.25) (layer "B.Cu") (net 27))
 (segment (start 131.445 146.5991) (end 133.5629 148.717) (width 0.25) (layer "B.Cu") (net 28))
 (segment (start 162.179 145.539) (end 162.179 140.973) (width 0.25) (layer "B.Cu") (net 28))
 (segment (start 133.5629 148.717) (end 159.001 148.717) (width 0.25) (layer "B.Cu") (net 28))
 (segment (start 159.001 148.717) (end 162.179 145.539) (width 0.25) (layer "B.Cu") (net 28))
 (segment (start 141.097 103.632) (end 156.083 118.618) (width 0.25) (layer "F.Cu") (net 15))
 (segment (start 129.794 103.632) (end 141.097 103.632) (width 0.25) (layer "F.Cu") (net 15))
 (segment (start 156.083 118.618) (end 156.083 135.509) (width 0.25) (layer "F.Cu") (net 15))
 (segment (start 156.083 135.509) (end 156.083 139.957) (width 0.25) (layer "F.Cu") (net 15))
 (segment (start 156.083 139.957) (end 159.639 143.513) (width 0.25) (layer "F.Cu") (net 15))
 (segment (start 154.81 110.744) (end 162.179 118.113) (width 0.25) (layer "B.Cu") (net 20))
 (segment (start 134.62 110.744) (end 154.81 110.744) (width 0.25) (layer "B.Cu") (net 20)))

